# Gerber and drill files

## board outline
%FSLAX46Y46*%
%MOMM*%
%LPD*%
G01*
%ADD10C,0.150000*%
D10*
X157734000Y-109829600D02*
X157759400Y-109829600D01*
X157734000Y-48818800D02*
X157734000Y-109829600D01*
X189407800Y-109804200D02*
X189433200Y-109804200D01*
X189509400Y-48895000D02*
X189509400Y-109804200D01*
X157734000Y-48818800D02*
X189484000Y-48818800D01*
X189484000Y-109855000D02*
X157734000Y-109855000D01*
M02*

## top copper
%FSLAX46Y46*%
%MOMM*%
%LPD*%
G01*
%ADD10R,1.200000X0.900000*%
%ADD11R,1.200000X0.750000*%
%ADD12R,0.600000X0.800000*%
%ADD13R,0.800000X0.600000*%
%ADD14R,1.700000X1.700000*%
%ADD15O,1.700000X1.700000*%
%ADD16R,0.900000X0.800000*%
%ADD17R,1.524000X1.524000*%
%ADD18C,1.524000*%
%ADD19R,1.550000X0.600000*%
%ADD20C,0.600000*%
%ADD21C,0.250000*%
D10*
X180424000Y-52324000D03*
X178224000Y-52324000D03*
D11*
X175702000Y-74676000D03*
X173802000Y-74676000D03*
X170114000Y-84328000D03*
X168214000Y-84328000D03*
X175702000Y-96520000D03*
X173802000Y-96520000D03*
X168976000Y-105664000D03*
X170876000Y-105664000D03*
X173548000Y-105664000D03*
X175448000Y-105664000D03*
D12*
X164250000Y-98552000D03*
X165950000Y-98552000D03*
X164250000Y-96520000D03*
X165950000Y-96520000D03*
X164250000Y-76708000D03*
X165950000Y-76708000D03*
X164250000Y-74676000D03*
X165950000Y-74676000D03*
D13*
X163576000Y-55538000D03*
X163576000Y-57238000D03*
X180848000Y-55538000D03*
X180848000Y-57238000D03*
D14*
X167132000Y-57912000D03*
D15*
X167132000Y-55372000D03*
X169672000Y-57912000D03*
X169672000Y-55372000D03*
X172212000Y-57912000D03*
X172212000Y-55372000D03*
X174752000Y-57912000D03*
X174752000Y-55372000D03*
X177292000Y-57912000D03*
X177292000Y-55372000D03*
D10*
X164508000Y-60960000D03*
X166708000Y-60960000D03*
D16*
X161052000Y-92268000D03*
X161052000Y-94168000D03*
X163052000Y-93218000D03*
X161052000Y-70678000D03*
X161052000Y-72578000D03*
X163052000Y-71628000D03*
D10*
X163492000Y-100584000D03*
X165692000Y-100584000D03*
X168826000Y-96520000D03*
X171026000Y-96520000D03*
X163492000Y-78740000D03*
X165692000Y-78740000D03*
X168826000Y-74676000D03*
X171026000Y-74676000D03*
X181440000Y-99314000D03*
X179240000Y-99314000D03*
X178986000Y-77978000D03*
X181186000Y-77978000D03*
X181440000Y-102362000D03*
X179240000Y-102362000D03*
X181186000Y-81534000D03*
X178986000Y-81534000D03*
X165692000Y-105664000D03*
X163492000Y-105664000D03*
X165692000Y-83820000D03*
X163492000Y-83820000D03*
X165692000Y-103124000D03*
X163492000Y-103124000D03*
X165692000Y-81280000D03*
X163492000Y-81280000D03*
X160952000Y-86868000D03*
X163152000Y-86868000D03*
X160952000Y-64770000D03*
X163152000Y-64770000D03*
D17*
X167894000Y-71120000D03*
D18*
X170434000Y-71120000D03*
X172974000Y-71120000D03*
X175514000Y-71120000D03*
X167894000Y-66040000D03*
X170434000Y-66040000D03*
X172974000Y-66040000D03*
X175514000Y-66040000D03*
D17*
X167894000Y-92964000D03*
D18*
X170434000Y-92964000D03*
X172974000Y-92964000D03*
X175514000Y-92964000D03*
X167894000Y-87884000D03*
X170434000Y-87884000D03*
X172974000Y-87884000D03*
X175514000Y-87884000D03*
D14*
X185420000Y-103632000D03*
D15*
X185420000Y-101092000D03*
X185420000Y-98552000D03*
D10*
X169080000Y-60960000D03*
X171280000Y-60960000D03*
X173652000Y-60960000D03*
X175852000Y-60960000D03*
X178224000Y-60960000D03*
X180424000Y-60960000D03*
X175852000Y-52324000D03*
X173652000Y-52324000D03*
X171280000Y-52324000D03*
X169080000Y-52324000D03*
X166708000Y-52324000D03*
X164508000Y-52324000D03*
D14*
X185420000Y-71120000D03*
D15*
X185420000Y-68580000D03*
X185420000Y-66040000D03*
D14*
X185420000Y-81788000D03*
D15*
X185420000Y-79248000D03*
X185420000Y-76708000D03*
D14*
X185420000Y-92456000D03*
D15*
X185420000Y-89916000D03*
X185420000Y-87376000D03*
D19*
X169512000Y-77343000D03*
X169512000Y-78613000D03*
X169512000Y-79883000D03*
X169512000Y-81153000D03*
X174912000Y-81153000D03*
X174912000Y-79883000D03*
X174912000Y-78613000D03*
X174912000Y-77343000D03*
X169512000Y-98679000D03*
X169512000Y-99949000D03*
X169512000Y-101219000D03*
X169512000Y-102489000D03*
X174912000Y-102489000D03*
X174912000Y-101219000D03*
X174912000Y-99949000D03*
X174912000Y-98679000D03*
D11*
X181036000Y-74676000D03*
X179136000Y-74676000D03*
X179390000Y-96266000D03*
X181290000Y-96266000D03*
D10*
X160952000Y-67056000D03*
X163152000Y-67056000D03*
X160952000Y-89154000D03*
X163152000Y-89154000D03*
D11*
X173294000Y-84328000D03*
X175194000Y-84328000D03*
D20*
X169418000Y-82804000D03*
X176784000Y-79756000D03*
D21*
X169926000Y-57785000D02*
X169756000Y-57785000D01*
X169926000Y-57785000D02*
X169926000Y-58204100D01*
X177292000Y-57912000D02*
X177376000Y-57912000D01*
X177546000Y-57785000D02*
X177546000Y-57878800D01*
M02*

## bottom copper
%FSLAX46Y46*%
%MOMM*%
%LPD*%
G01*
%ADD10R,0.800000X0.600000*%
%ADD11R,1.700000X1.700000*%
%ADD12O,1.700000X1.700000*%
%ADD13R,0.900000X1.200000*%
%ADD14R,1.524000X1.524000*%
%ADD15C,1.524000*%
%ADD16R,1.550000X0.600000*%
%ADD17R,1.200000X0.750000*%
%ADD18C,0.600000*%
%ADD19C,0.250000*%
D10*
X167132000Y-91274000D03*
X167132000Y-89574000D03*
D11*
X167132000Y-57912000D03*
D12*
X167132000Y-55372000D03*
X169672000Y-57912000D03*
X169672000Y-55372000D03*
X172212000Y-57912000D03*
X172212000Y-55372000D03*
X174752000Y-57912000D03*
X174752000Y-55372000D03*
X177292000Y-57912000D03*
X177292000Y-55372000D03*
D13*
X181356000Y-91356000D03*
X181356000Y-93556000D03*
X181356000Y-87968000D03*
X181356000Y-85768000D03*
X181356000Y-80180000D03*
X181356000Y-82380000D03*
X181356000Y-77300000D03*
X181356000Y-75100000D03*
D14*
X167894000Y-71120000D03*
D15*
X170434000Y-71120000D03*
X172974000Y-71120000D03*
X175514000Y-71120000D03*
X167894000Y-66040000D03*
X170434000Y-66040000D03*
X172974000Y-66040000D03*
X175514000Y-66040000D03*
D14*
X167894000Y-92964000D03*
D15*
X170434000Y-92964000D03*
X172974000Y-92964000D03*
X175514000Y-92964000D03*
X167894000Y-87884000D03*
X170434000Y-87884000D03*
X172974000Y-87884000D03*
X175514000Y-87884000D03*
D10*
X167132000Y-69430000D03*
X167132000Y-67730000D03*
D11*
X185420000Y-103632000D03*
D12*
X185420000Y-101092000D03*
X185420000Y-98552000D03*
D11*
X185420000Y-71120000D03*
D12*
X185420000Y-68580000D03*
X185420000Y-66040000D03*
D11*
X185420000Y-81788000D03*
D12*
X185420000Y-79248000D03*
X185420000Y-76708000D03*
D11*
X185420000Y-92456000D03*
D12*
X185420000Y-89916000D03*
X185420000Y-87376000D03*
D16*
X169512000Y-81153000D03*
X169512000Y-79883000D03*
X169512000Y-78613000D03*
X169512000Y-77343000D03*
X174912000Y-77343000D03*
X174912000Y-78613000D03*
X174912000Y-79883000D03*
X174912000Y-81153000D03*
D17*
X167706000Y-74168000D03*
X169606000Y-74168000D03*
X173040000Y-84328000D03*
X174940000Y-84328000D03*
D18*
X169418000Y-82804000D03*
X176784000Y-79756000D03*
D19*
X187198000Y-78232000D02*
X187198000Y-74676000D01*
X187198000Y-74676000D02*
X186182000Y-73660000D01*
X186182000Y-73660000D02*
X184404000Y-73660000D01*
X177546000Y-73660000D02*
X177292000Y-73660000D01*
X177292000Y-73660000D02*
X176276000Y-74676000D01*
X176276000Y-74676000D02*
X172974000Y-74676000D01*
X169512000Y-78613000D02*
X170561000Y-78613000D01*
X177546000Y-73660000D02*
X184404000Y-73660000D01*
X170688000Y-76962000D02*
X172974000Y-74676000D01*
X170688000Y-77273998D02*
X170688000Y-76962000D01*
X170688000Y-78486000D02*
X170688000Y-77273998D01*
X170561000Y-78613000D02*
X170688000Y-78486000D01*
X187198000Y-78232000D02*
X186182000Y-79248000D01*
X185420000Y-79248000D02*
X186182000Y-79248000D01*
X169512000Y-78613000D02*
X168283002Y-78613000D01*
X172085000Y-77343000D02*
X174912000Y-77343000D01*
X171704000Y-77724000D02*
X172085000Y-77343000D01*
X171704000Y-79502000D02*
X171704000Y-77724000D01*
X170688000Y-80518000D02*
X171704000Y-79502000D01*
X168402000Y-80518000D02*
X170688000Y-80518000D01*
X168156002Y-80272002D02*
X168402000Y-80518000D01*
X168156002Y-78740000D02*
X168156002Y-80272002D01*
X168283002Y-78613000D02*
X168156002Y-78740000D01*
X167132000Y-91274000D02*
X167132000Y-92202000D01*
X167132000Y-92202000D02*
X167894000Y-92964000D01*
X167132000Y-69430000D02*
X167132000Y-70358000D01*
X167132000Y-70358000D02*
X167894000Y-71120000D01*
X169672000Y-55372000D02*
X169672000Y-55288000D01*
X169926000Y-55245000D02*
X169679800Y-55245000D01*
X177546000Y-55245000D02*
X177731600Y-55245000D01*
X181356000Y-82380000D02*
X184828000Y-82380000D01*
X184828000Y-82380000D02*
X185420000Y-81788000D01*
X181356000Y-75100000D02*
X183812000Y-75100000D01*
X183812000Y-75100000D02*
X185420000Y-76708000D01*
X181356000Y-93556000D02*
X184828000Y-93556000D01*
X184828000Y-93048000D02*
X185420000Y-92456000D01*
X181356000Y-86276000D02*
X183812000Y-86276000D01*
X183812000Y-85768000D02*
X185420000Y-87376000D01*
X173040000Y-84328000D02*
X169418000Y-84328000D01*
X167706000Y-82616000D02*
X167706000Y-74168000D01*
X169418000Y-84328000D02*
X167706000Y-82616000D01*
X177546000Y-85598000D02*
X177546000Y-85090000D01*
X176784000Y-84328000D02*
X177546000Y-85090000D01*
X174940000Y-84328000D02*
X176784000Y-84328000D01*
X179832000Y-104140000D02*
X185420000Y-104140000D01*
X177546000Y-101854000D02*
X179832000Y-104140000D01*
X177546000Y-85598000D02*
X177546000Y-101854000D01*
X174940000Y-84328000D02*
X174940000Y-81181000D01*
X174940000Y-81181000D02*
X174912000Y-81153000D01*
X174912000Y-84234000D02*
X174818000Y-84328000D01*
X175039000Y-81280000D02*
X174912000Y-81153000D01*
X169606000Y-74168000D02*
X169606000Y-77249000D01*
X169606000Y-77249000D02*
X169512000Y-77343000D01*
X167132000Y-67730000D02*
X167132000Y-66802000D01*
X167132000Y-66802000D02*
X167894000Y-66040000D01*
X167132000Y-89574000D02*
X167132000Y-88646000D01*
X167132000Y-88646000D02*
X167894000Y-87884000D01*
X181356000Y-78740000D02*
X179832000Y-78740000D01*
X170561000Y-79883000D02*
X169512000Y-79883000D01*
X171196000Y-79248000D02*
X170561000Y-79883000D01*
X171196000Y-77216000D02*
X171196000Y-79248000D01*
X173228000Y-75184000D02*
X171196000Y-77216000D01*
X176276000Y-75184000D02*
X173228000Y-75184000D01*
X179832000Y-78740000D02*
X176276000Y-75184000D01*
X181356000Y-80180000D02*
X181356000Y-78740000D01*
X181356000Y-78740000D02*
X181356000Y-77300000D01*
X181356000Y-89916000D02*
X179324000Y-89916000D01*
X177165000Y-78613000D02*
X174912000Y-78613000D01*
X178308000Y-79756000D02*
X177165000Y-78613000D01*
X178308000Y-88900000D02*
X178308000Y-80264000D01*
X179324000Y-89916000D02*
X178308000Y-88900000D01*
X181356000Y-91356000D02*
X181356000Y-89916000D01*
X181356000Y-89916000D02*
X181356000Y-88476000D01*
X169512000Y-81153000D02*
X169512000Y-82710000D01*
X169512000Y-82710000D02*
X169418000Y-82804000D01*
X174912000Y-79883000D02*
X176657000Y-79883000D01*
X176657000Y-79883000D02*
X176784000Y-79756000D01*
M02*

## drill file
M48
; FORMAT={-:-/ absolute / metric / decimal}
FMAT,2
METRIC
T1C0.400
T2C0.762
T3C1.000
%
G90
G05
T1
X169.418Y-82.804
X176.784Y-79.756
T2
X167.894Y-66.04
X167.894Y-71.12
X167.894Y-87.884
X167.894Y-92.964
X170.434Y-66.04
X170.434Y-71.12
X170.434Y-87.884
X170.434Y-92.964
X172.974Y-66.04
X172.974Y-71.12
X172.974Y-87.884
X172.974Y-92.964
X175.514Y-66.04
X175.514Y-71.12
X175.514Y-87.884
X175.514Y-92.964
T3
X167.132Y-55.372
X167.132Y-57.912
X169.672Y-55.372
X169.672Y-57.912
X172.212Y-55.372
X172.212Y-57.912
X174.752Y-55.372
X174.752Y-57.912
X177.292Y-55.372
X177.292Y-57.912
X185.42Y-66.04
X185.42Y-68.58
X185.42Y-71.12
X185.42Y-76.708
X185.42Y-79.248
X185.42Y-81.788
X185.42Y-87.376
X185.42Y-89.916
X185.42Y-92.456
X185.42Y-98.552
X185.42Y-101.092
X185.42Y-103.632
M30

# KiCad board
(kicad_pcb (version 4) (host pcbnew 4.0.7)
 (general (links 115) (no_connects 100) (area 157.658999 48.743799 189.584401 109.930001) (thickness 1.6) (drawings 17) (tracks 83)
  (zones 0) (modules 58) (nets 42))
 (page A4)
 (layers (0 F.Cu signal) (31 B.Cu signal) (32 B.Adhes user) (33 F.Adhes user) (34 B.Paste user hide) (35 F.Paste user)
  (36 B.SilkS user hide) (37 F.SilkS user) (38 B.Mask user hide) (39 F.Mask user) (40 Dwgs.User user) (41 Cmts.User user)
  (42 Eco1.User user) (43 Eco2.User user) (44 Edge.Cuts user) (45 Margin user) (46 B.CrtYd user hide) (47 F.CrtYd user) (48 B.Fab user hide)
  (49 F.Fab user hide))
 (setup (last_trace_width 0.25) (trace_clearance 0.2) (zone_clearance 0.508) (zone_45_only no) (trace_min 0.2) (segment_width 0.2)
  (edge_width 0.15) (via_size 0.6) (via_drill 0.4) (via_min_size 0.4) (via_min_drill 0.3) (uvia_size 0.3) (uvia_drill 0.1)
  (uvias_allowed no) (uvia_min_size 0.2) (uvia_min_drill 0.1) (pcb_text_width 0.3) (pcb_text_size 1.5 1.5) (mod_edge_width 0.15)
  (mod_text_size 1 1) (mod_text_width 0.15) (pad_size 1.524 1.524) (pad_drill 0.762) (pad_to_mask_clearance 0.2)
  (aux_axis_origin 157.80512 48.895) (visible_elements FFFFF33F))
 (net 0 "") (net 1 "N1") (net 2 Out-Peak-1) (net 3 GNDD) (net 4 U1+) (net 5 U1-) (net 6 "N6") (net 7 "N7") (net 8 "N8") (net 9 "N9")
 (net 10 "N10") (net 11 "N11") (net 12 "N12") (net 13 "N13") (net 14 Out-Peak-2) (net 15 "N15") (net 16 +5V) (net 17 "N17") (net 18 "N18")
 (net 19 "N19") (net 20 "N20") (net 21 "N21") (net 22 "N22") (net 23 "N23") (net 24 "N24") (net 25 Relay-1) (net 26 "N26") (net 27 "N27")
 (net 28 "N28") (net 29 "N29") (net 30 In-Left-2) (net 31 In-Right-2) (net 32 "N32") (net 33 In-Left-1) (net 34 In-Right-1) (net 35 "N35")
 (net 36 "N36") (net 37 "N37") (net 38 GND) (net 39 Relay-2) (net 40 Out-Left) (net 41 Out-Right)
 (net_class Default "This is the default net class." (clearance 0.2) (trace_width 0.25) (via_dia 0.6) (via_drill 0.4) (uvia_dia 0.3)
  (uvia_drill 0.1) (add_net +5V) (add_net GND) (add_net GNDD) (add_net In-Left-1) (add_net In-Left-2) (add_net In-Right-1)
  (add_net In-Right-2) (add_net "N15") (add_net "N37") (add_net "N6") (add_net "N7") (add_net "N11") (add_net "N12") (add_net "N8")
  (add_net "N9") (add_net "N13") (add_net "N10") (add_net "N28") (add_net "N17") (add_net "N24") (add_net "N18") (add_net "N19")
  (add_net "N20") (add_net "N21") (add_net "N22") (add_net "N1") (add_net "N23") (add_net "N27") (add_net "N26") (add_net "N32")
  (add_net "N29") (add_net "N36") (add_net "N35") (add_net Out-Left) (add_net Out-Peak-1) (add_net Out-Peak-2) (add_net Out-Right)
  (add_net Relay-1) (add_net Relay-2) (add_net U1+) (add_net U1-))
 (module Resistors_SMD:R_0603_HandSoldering (layer F.Cu) (at 179.324 52.324 180)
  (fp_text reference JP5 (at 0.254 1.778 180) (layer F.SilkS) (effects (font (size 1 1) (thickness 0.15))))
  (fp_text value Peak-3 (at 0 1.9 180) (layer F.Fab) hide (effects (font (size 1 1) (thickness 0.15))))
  (pad 1 smd rect (at -1.1 0 180) (size 1.2 0.9) (layers F.Cu F.Paste F.Mask) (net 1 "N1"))
  (pad 2 smd rect (at 1.1 0 180) (size 1.2 0.9) (layers F.Cu F.Paste F.Mask) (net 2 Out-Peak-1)))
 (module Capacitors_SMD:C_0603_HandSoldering (layer F.Cu) (at 174.752 74.676 180)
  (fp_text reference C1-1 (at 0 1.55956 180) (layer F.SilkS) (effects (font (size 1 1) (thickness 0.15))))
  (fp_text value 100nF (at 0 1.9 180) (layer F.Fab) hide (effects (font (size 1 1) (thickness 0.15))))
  (pad 1 smd rect (at -0.95 0 180) (size 1.2 0.75) (layers F.Cu F.Paste F.Mask) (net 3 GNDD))
  (pad 2 smd rect (at 0.95 0 180) (size 1.2 0.75) (layers F.Cu F.Paste F.Mask) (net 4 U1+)))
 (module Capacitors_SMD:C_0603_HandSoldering (layer F.Cu) (at 169.164 84.328 180)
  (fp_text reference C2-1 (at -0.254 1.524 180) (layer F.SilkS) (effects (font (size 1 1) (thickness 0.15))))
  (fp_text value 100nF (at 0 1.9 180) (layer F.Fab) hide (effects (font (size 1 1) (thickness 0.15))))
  (pad 1 smd rect (at -0.95 0 180) (size 1.2 0.75) (layers F.Cu F.Paste F.Mask) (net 3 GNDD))
  (pad 2 smd rect (at 0.95 0 180) (size 1.2 0.75) (layers F.Cu F.Paste F.Mask) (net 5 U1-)))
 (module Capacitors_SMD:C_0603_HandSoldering (layer F.Cu) (at 174.752 96.52 180)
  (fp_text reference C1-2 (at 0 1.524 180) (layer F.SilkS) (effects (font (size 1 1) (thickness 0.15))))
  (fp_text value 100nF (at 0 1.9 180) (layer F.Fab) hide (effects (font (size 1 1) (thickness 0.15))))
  (pad 1 smd rect (at -0.95 0 180) (size 1.2 0.75) (layers F.Cu F.Paste F.Mask) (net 3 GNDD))
  (pad 2 smd rect (at 0.95 0 180) (size 1.2 0.75) (layers F.Cu F.Paste F.Mask) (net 4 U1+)))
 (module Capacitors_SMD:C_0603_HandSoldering (layer F.Cu) (at 169.926 105.664)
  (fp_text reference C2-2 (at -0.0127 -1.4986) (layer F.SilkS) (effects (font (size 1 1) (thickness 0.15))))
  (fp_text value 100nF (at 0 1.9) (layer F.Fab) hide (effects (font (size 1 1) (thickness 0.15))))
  (pad 1 smd rect (at -0.95 0) (size 1.2 0.75) (layers F.Cu F.Paste F.Mask) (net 3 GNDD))
  (pad 2 smd rect (at 0.95 0) (size 1.2 0.75) (layers F.Cu F.Paste F.Mask) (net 5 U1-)))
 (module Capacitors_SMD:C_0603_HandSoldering (layer F.Cu) (at 174.498 105.664)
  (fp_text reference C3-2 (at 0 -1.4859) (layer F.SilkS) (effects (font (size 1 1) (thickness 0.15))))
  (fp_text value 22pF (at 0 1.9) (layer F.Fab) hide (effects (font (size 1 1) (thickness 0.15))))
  (pad 1 smd rect (at -0.95 0) (size 1.2 0.75) (layers F.Cu F.Paste F.Mask) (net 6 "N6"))
  (pad 2 smd rect (at 0.95 0) (size 1.2 0.75) (layers F.Cu F.Paste F.Mask) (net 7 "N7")))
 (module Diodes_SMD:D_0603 (layer F.Cu) (at 165.1 98.552)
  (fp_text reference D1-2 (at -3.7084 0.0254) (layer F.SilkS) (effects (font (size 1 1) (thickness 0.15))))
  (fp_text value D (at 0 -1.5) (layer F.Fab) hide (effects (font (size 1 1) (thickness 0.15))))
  (pad 1 smd rect (at -0.85 0) (size 0.6 0.8) (layers F.Cu F.Paste F.Mask) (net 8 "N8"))
  (pad 2 smd rect (at 0.85 0) (size 0.6 0.8) (layers F.Cu F.Paste F.Mask) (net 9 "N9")))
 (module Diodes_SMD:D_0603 (layer F.Cu) (at 165.1 96.52)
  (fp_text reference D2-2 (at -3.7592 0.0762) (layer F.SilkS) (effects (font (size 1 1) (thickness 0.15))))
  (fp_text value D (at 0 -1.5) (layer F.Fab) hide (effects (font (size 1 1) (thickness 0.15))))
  (pad 1 smd rect (at -0.85 0) (size 0.6 0.8) (layers F.Cu F.Paste F.Mask) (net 9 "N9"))
  (pad 2 smd rect (at 0.85 0) (size 0.6 0.8) (layers F.Cu F.Paste F.Mask) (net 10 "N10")))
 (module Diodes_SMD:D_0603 (layer F.Cu) (at 165.1 76.708)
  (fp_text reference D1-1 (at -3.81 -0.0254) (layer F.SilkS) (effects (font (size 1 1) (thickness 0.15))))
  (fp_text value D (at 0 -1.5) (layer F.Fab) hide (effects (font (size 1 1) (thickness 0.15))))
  (pad 1 smd rect (at -0.85 0) (size 0.6 0.8) (layers F.Cu F.Paste F.Mask) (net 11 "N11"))
  (pad 2 smd rect (at 0.85 0) (size 0.6 0.8) (layers F.Cu F.Paste F.Mask) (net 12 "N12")))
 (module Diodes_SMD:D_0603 (layer F.Cu) (at 165.1 74.676)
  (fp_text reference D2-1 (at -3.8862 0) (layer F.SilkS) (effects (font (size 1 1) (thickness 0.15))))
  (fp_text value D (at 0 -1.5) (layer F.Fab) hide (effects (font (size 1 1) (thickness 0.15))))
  (pad 1 smd rect (at -0.85 0) (size 0.6 0.8) (layers F.Cu F.Paste F.Mask) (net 12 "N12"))
  (pad 2 smd rect (at 0.85 0) (size 0.6 0.8) (layers F.Cu F.Paste F.Mask) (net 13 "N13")))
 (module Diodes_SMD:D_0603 (layer F.Cu) (at 163.576 56.388 270)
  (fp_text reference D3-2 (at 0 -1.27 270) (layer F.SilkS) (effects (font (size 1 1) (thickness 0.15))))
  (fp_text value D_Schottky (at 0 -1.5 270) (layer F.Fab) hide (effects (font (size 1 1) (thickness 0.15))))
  (pad 1 smd rect (at -0.85 0 270) (size 0.6 0.8) (layers F.Cu F.Paste F.Mask) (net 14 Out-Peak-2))
  (pad 2 smd rect (at 0.85 0 270) (size 0.6 0.8) (layers F.Cu F.Paste F.Mask) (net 6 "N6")))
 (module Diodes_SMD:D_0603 (layer F.Cu) (at 180.848 56.388 270)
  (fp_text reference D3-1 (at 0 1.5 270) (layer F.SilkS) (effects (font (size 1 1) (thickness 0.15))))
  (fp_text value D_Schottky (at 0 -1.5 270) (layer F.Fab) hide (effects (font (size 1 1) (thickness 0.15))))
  (pad 1 smd rect (at -0.85 0 270) (size 0.6 0.8) (layers F.Cu F.Paste F.Mask) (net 2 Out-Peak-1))
  (pad 2 smd rect (at 0.85 0 270) (size 0.6 0.8) (layers F.Cu F.Paste F.Mask) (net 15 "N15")))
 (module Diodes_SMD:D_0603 (layer B.Cu) (at 167.132 90.424 90)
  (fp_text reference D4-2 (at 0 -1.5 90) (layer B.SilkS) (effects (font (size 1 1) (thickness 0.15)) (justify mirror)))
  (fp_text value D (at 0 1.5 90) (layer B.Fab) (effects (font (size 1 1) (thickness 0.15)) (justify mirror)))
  (pad 1 smd rect (at -0.85 0 90) (size 0.6 0.8) (layers B.Cu B.Paste B.Mask) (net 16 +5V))
  (pad 2 smd rect (at 0.85 0 90) (size 0.6 0.8) (layers B.Cu B.Paste B.Mask) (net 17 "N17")))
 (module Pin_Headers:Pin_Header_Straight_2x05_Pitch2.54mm (layer F.Cu) (at 167.132 57.912 90)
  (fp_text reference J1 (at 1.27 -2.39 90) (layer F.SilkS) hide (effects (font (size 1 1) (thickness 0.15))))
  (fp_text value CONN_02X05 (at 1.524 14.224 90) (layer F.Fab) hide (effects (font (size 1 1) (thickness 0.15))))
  (pad 1 thru_hole rect (at 0 0 90) (size 1.7 1.7) (drill 1) (layers *.Cu *.Mask) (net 16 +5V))
  (pad 2 thru_hole oval (at 2.54 0 90) (size 1.7 1.7) (drill 1) (layers *.Cu *.Mask) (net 3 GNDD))
  (pad 3 thru_hole oval (at 0 2.54 90) (size 1.7 1.7) (drill 1) (layers *.Cu *.Mask) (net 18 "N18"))
  (pad 4 thru_hole oval (at 2.54 2.54 90) (size 1.7 1.7) (drill 1) (layers *.Cu *.Mask) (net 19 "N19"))
  (pad 5 thru_hole oval (at 0 5.08 90) (size 1.7 1.7) (drill 1) (layers *.Cu *.Mask) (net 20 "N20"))
  (pad 6 thru_hole oval (at 2.54 5.08 90) (size 1.7 1.7) (drill 1) (layers *.Cu *.Mask) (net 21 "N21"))
  (pad 7 thru_hole oval (at 0 7.62 90) (size 1.7 1.7) (drill 1) (layers *.Cu *.Mask) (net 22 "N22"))
  (pad 8 thru_hole oval (at 2.54 7.62 90) (size 1.7 1.7) (drill 1) (layers *.Cu *.Mask) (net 1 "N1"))
  (pad 9 thru_hole oval (at 0 10.16 90) (size 1.7 1.7) (drill 1) (layers *.Cu *.Mask) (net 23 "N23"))
  (pad 10 thru_hole oval (at 2.54 10.16 90) (size 1.7 1.7) (drill 1) (layers *.Cu *.Mask) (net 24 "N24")))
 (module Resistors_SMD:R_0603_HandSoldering (layer F.Cu) (at 165.608 60.96)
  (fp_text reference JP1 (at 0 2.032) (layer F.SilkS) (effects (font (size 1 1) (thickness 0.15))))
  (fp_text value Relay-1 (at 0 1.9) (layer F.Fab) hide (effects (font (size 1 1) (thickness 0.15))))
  (pad 1 smd rect (at -1.1 0) (size 1.2 0.9) (layers F.Cu F.Paste F.Mask) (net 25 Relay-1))
  (pad 2 smd rect (at 1.1 0) (size 1.2 0.9) (layers F.Cu F.Paste F.Mask) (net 18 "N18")))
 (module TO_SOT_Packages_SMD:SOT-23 (layer F.Cu) (at 162.052 93.218)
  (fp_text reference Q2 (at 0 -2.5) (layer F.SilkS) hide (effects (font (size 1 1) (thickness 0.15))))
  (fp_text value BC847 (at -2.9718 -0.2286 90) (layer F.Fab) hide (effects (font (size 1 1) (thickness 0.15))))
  (pad 1 smd rect (at -1 -0.95) (size 0.9 0.8) (layers F.Cu F.Paste F.Mask) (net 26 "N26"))
  (pad 2 smd rect (at -1 0.95) (size 0.9 0.8) (layers F.Cu F.Paste F.Mask) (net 3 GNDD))
  (pad 3 smd rect (at 1 0) (size 0.9 0.8) (layers F.Cu F.Paste F.Mask) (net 17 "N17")))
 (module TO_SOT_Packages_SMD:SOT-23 (layer F.Cu) (at 162.052 71.628)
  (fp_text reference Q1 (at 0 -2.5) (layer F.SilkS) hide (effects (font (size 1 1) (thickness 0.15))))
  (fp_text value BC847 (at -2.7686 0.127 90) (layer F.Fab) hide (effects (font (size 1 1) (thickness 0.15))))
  (pad 1 smd rect (at -1 -0.95) (size 0.9 0.8) (layers F.Cu F.Paste F.Mask) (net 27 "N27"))
  (pad 2 smd rect (at -1 0.95) (size 0.9 0.8) (layers F.Cu F.Paste F.Mask) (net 3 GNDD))
  (pad 3 smd rect (at 1 0) (size 0.9 0.8) (layers F.Cu F.Paste F.Mask) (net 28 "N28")))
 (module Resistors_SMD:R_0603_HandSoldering (layer B.Cu) (at 181.356 92.456 270)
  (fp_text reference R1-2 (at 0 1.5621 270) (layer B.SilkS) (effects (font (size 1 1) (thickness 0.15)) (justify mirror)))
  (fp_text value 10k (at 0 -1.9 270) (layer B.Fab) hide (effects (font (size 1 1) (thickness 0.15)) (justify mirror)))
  (pad 1 smd rect (at -1.1 0 270) (size 1.2 0.9) (layers B.Cu B.Paste B.Mask) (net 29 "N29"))
  (pad 2 smd rect (at 1.1 0 270) (size 1.2 0.9) (layers B.Cu B.Paste B.Mask) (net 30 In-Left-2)))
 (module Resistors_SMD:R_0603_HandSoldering (layer B.Cu) (at 181.356 86.868 90)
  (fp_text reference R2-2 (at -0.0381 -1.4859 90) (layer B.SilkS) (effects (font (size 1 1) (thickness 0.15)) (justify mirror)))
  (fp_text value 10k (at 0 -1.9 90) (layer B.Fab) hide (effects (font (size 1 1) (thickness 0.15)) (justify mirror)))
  (pad 1 smd rect (at -1.1 0 90) (size 1.2 0.9) (layers B.Cu B.Paste B.Mask) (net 29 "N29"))
  (pad 2 smd rect (at 1.1 0 90) (size 1.2 0.9) (layers B.Cu B.Paste B.Mask) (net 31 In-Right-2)))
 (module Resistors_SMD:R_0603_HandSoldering (layer B.Cu) (at 181.356 81.28 270)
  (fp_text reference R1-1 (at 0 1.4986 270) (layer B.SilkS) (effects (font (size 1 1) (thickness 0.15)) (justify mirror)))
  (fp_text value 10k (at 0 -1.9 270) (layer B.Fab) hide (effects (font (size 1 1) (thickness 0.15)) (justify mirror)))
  (pad 1 smd rect (at -1.1 0 270) (size 1.2 0.9) (layers B.Cu B.Paste B.Mask) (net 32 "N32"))
  (pad 2 smd rect (at 1.1 0 270) (size 1.2 0.9) (layers B.Cu B.Paste B.Mask) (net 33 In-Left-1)))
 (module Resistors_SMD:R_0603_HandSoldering (layer B.Cu) (at 181.356 76.2 90)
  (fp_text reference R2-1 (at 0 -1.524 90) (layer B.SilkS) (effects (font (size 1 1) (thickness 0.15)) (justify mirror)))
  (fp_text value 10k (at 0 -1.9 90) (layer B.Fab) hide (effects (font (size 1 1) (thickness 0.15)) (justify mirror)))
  (pad 1 smd rect (at -1.1 0 90) (size 1.2 0.9) (layers B.Cu B.Paste B.Mask) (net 32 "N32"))
  (pad 2 smd rect (at 1.1 0 90) (size 1.2 0.9) (layers B.Cu B.Paste B.Mask) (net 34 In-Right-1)))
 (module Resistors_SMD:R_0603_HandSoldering (layer F.Cu) (at 164.592 100.584)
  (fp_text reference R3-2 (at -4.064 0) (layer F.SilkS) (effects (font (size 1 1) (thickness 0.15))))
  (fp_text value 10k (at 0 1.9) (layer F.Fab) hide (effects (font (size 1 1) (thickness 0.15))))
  (pad 1 smd rect (at -1.1 0) (size 1.2 0.9) (layers F.Cu F.Paste F.Mask) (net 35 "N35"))
  (pad 2 smd rect (at 1.1 0) (size 1.2 0.9) (layers F.Cu F.Paste F.Mask) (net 29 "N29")))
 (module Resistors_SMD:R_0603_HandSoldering (layer F.Cu) (at 169.926 96.52)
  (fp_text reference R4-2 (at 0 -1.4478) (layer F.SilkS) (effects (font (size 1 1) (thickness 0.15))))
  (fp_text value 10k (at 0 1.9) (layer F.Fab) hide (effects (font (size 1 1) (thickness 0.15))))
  (pad 1 smd rect (at -1.1 0) (size 1.2 0.9) (layers F.Cu F.Paste F.Mask) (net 8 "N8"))
  (pad 2 smd rect (at 1.1 0) (size 1.2 0.9) (layers F.Cu F.Paste F.Mask) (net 35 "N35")))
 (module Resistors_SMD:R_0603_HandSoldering (layer F.Cu) (at 164.592 78.74)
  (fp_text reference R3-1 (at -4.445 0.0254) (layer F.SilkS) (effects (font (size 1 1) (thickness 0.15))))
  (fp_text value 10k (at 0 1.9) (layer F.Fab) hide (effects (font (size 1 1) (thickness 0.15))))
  (pad 1 smd rect (at -1.1 0) (size 1.2 0.9) (layers F.Cu F.Paste F.Mask) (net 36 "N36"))
  (pad 2 smd rect (at 1.1 0) (size 1.2 0.9) (layers F.Cu F.Paste F.Mask) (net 32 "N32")))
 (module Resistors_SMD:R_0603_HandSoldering (layer F.Cu) (at 169.926 74.676)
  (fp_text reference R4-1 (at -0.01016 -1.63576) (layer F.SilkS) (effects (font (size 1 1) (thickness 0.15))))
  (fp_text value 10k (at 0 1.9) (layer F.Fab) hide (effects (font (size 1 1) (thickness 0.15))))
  (pad 1 smd rect (at -1.1 0) (size 1.2 0.9) (layers F.Cu F.Paste F.Mask) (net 11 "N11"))
  (pad 2 smd rect (at 1.1 0) (size 1.2 0.9) (layers F.Cu F.Paste F.Mask) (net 36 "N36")))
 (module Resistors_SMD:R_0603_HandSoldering (layer F.Cu) (at 180.34 99.314 180)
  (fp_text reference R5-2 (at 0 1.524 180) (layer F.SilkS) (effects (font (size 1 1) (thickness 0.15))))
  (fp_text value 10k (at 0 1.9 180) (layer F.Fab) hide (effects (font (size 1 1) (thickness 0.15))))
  (pad 1 smd rect (at -1.1 0 180) (size 1.2 0.9) (layers F.Cu F.Paste F.Mask) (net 10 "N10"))
  (pad 2 smd rect (at 1.1 0 180) (size 1.2 0.9) (layers F.Cu F.Paste F.Mask) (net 35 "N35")))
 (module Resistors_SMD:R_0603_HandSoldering (layer F.Cu) (at 180.086 77.978)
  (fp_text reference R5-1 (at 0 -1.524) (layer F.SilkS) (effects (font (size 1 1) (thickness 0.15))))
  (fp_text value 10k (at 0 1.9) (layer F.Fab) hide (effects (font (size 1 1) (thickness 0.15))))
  (pad 1 smd rect (at -1.1 0) (size 1.2 0.9) (layers F.Cu F.Paste F.Mask) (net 13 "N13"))
  (pad 2 smd rect (at 1.1 0) (size 1.2 0.9) (layers F.Cu F.Paste F.Mask) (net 36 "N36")))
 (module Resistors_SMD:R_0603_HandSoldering (layer F.Cu) (at 180.34 102.362 180)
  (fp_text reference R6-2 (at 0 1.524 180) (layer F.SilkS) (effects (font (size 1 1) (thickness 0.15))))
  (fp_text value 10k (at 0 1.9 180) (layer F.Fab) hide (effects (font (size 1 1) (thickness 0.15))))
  (pad 1 smd rect (at -1.1 0 180) (size 1.2 0.9) (layers F.Cu F.Paste F.Mask) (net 7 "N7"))
  (pad 2 smd rect (at 1.1 0 180) (size 1.2 0.9) (layers F.Cu F.Paste F.Mask) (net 10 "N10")))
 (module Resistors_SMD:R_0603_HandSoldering (layer F.Cu) (at 180.086 81.534 180)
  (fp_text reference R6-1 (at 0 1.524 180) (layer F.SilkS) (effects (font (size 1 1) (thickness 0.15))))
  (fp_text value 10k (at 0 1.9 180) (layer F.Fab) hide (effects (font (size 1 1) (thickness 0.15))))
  (pad 1 smd rect (at -1.1 0 180) (size 1.2 0.9) (layers F.Cu F.Paste F.Mask) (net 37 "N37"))
  (pad 2 smd rect (at 1.1 0 180) (size 1.2 0.9) (layers F.Cu F.Paste F.Mask) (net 13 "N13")))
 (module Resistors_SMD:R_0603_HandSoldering (layer F.Cu) (at 164.592 105.664 180)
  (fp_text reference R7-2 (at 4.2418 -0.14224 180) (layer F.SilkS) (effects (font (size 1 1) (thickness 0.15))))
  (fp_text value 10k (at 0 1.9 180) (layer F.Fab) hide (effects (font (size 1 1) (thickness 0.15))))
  (pad 1 smd rect (at -1.1 0 180) (size 1.2 0.9) (layers F.Cu F.Paste F.Mask) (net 6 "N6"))
  (pad 2 smd rect (at 1.1 0 180) (size 1.2 0.9) (layers F.Cu F.Paste F.Mask) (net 7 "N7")))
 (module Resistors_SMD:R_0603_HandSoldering (layer F.Cu) (at 164.592 83.82 180)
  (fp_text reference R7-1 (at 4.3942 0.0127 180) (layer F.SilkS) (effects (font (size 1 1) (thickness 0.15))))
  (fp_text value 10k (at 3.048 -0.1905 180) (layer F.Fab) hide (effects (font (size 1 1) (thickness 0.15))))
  (pad 1 smd rect (at -1.1 0 180) (size 1.2 0.9) (layers F.Cu F.Paste F.Mask) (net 15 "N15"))
  (pad 2 smd rect (at 1.1 0 180) (size 1.2 0.9) (layers F.Cu F.Paste F.Mask) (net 37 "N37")))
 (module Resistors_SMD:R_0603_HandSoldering (layer F.Cu) (at 164.592 103.124 180)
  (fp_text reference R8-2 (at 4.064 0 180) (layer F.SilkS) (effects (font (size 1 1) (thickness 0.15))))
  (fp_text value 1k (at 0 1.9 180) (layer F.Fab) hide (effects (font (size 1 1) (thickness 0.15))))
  (pad 1 smd rect (at -1.1 0 180) (size 1.2 0.9) (layers F.Cu F.Paste F.Mask) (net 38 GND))
  (pad 2 smd rect (at 1.1 0 180) (size 1.2 0.9) (layers F.Cu F.Paste F.Mask) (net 14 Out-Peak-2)))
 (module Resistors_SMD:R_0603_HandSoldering (layer F.Cu) (at 164.592 81.28 180)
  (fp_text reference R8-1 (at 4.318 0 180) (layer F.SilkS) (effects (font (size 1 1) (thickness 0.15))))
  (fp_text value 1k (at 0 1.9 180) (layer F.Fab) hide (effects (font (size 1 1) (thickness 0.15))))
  (pad 1 smd rect (at -1.1 0 180) (size 1.2 0.9) (layers F.Cu F.Paste F.Mask) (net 38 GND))
  (pad 2 smd rect (at 1.1 0 180) (size 1.2 0.9) (layers F.Cu F.Paste F.Mask) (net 2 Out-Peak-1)))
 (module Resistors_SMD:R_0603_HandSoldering (layer F.Cu) (at 162.052 86.868)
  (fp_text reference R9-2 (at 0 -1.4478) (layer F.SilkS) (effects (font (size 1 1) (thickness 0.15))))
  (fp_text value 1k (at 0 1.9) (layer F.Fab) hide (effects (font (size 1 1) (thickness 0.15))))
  (pad 1 smd rect (at -1.1 0) (size 1.2 0.9) (layers F.Cu F.Paste F.Mask) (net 26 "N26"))
  (pad 2 smd rect (at 1.1 0) (size 1.2 0.9) (layers F.Cu F.Paste F.Mask) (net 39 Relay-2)))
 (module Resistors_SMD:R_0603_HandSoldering (layer F.Cu) (at 162.052 64.77)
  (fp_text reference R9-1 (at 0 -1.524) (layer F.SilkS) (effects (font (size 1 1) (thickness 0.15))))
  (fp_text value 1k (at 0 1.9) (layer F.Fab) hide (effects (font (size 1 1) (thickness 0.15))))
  (pad 1 smd rect (at -1.1 0) (size 1.2 0.9) (layers F.Cu F.Paste F.Mask) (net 27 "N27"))
  (pad 2 smd rect (at 1.1 0) (size 1.2 0.9) (layers F.Cu F.Paste F.Mask) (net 25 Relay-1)))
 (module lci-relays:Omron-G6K (layer F.Cu) (at 171.704 68.58)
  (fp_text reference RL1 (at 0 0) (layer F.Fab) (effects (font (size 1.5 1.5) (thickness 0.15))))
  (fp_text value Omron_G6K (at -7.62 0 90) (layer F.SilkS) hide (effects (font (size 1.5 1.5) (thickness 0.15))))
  (pad 1 thru_hole rect (at -3.81 2.54) (size 1.524 1.524) (drill 0.762) (layers *.Cu *.Mask F.SilkS) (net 16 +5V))
  (pad 2 thru_hole circle (at -1.27 2.54) (size 1.524 1.524) (drill 0.762) (layers *.Cu *.Mask F.SilkS))
  (pad 3 thru_hole circle (at 1.27 2.54) (size 1.524 1.524) (drill 0.762) (layers *.Cu *.Mask F.SilkS) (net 33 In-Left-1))
  (pad 4 thru_hole circle (at 3.81 2.54) (size 1.524 1.524) (drill 0.762) (layers *.Cu *.Mask F.SilkS) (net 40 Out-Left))
  (pad 8 thru_hole circle (at -3.81 -2.54) (size 1.524 1.524) (drill 0.762) (layers *.Cu *.Mask F.SilkS) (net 28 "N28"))
  (pad 7 thru_hole circle (at -1.27 -2.54) (size 1.524 1.524) (drill 0.762) (layers *.Cu *.Mask F.SilkS))
  (pad 6 thru_hole circle (at 1.27 -2.54) (size 1.524 1.524) (drill 0.762) (layers *.Cu *.Mask F.SilkS) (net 34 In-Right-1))
  (pad 5 thru_hole circle (at 3.81 -2.54) (size 1.524 1.524) (drill 0.762) (layers *.Cu *.Mask F.SilkS) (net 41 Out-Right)))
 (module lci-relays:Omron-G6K (layer F.Cu) (at 171.704 90.424)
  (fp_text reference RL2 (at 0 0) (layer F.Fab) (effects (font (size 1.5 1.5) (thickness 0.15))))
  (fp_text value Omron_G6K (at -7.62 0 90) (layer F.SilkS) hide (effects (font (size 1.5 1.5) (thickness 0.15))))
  (pad 1 thru_hole rect (at -3.81 2.54) (size 1.524 1.524) (drill 0.762) (layers *.Cu *.Mask F.SilkS) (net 16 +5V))
  (pad 2 thru_hole circle (at -1.27 2.54) (size 1.524 1.524) (drill 0.762) (layers *.Cu *.Mask F.SilkS))
  (pad 3 thru_hole circle (at 1.27 2.54) (size 1.524 1.524) (drill 0.762) (layers *.Cu *.Mask F.SilkS) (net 30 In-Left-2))
  (pad 4 thru_hole circle (at 3.81 2.54) (size 1.524 1.524) (drill 0.762) (layers *.Cu *.Mask F.SilkS) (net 40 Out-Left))
  (pad 8 thru_hole circle (at -3.81 -2.54) (size 1.524 1.524) (drill 0.762) (layers *.Cu *.Mask F.SilkS) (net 17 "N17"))
  (pad 7 thru_hole circle (at -1.27 -2.54) (size 1.524 1.524) (drill 0.762) (layers *.Cu *.Mask F.SilkS))
  (pad 6 thru_hole circle (at 1.27 -2.54) (size 1.524 1.524) (drill 0.762) (layers *.Cu *.Mask F.SilkS) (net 31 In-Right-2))
  (pad 5 thru_hole circle (at 3.81 -2.54) (size 1.524 1.524) (drill 0.762) (layers *.Cu *.Mask F.SilkS) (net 41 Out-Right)))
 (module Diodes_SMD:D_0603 (layer B.Cu) (at 167.132 68.58 90)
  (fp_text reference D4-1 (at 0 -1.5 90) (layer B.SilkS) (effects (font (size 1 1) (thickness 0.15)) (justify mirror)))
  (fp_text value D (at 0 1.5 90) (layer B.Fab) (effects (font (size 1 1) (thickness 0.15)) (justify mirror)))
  (pad 1 smd rect (at -0.85 0 90) (size 0.6 0.8) (layers B.Cu B.Paste B.Mask) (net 16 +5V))
  (pad 2 smd rect (at 0.85 0 90) (size 0.6 0.8) (layers B.Cu B.Paste B.Mask) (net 28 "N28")))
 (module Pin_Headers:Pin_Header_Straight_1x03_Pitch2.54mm (layer F.Cu) (at 185.42 103.632 180)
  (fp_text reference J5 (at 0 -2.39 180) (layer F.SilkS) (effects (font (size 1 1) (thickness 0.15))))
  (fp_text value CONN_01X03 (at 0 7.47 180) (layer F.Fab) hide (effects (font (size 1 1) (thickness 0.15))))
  (pad 1 thru_hole rect (at 0 0 180) (size 1.7 1.7) (drill 1) (layers *.Cu *.Mask) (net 4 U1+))
  (pad 2 thru_hole oval (at 0 2.54 180) (size 1.7 1.7) (drill 1) (layers *.Cu *.Mask) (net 3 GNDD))
  (pad 3 thru_hole oval (at 0 5.08 180) (size 1.7 1.7) (drill 1) (layers *.Cu *.Mask) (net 5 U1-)))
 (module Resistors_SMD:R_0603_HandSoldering (layer F.Cu) (at 170.18 60.96)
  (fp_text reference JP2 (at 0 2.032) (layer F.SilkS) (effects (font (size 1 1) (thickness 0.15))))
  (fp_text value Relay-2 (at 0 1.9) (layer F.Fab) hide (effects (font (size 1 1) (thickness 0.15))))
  (pad 1 smd rect (at -1.1 0) (size 1.2 0.9) (layers F.Cu F.Paste F.Mask) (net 39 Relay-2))
  (pad 2 smd rect (at 1.1 0) (size 1.2 0.9) (layers F.Cu F.Paste F.Mask) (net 20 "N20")))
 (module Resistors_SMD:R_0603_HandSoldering (layer F.Cu) (at 174.752 60.96)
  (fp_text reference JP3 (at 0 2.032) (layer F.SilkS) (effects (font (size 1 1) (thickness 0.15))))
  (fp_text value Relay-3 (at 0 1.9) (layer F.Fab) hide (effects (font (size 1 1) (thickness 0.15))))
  (pad 1 smd rect (at -1.1 0) (size 1.2 0.9) (layers F.Cu F.Paste F.Mask) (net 25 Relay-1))
  (pad 2 smd rect (at 1.1 0) (size 1.2 0.9) (layers F.Cu F.Paste F.Mask) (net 22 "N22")))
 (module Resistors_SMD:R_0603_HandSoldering (layer F.Cu) (at 179.324 60.96)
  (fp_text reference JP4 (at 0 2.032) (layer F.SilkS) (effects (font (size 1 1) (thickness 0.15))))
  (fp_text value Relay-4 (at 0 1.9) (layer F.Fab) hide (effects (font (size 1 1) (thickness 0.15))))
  (pad 1 smd rect (at -1.1 0) (size 1.2 0.9) (layers F.Cu F.Paste F.Mask) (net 39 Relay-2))
  (pad 2 smd rect (at 1.1 0) (size 1.2 0.9) (layers F.Cu F.Paste F.Mask) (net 23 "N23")))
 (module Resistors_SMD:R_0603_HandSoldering (layer F.Cu) (at 174.752 52.324 180)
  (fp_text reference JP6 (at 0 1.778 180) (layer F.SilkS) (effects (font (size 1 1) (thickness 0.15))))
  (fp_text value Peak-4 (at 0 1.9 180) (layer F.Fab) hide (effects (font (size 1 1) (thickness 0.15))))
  (pad 1 smd rect (at -1.1 0 180) (size 1.2 0.9) (layers F.Cu F.Paste F.Mask) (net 24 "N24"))
  (pad 2 smd rect (at 1.1 0 180) (size 1.2 0.9) (layers F.Cu F.Paste F.Mask) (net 14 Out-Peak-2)))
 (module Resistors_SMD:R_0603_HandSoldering (layer F.Cu) (at 170.18 52.324 180)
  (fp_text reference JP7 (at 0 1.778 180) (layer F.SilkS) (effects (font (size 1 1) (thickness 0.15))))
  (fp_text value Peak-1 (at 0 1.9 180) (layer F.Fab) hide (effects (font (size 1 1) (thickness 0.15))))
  (pad 1 smd rect (at -1.1 0 180) (size 1.2 0.9) (layers F.Cu F.Paste F.Mask) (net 19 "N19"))
  (pad 2 smd rect (at 1.1 0 180) (size 1.2 0.9) (layers F.Cu F.Paste F.Mask) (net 2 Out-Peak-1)))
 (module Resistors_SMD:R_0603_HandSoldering (layer F.Cu) (at 165.608 52.324 180)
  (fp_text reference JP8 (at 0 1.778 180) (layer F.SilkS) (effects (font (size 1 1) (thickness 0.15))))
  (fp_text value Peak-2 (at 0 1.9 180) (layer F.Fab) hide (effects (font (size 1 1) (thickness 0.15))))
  (pad 1 smd rect (at -1.1 0 180) (size 1.2 0.9) (layers F.Cu F.Paste F.Mask) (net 21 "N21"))
  (pad 2 smd rect (at 1.1 0 180) (size 1.2 0.9) (layers F.Cu F.Paste F.Mask) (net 14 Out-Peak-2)))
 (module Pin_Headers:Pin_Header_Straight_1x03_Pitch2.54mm (layer F.Cu) (at 185.42 71.12 180)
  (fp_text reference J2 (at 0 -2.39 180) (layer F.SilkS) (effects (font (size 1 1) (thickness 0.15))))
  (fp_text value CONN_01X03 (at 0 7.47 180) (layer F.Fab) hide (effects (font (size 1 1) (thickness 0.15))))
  (pad 1 thru_hole rect (at 0 0 180) (size 1.7 1.7) (drill 1) (layers *.Cu *.Mask) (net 41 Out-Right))
  (pad 2 thru_hole oval (at 0 2.54 180) (size 1.7 1.7) (drill 1) (layers *.Cu *.Mask) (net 38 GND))
  (pad 3 thru_hole oval (at 0 5.08 180) (size 1.7 1.7) (drill 1) (layers *.Cu *.Mask) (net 40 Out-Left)))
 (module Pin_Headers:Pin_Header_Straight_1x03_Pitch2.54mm (layer F.Cu) (at 185.42 81.788 180)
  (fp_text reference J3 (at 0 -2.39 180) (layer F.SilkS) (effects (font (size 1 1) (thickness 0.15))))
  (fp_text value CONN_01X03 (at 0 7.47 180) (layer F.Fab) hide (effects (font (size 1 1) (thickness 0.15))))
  (pad 1 thru_hole rect (at 0 0 180) (size 1.7 1.7) (drill 1) (layers *.Cu *.Mask) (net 33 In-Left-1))
  (pad 2 thru_hole oval (at 0 2.54 180) (size 1.7 1.7) (drill 1) (layers *.Cu *.Mask) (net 38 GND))
  (pad 3 thru_hole oval (at 0 5.08 180) (size 1.7 1.7) (drill 1) (layers *.Cu *.Mask) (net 34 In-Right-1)))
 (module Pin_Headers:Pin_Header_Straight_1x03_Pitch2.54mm (layer F.Cu) (at 185.42 92.456 180)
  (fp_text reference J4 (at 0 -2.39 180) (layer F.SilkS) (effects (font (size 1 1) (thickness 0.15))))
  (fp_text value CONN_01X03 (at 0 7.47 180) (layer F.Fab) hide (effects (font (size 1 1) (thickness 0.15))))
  (pad 1 thru_hole rect (at 0 0 180) (size 1.7 1.7) (drill 1) (layers *.Cu *.Mask) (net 30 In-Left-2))
  (pad 2 thru_hole oval (at 0 2.54 180) (size 1.7 1.7) (drill 1) (layers *.Cu *.Mask) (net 38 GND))
  (pad 3 thru_hole oval (at 0 5.08 180) (size 1.7 1.7) (drill 1) (layers *.Cu *.Mask) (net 31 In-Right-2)))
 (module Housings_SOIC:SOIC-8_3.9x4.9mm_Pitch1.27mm (layer B.Cu) (at 172.212 79.248)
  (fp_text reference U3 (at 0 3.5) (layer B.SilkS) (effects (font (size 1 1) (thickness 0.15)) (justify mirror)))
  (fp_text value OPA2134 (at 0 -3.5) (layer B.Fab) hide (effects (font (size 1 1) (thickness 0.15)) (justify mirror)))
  (pad 1 smd rect (at -2.7 1.905) (size 1.55 0.6) (layers B.Cu B.Paste B.Mask) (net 36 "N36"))
  (pad 2 smd rect (at -2.7 0.635) (size 1.55 0.6) (layers B.Cu B.Paste B.Mask) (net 32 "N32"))
  (pad 3 smd rect (at -2.7 -0.635) (size 1.55 0.6) (layers B.Cu B.Paste B.Mask) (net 38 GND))
  (pad 4 smd rect (at -2.7 -1.905) (size 1.55 0.6) (layers B.Cu B.Paste B.Mask) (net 5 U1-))
  (pad 5 smd rect (at 2.7 -1.905) (size 1.55 0.6) (layers B.Cu B.Paste B.Mask) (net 38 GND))
  (pad 6 smd rect (at 2.7 -0.635) (size 1.55 0.6) (layers B.Cu B.Paste B.Mask) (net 29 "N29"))
  (pad 7 smd rect (at 2.7 0.635) (size 1.55 0.6) (layers B.Cu B.Paste B.Mask) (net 35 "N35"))
  (pad 8 smd rect (at 2.7 1.905) (size 1.55 0.6) (layers B.Cu B.Paste B.Mask) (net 4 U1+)))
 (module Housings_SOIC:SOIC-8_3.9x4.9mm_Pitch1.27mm (layer F.Cu) (at 172.212 79.248)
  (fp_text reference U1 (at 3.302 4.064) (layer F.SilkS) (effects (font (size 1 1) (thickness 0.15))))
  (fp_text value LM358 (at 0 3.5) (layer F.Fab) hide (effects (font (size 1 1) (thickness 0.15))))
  (pad 1 smd rect (at -2.7 -1.905) (size 1.55 0.6) (layers F.Cu F.Paste F.Mask) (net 12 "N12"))
  (pad 2 smd rect (at -2.7 -0.635) (size 1.55 0.6) (layers F.Cu F.Paste F.Mask) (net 36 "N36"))
  (pad 3 smd rect (at -2.7 0.635) (size 1.55 0.6) (layers F.Cu F.Paste F.Mask) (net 38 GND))
  (pad 4 smd rect (at -2.7 1.905) (size 1.55 0.6) (layers F.Cu F.Paste F.Mask) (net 5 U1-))
  (pad 5 smd rect (at 2.7 1.905) (size 1.55 0.6) (layers F.Cu F.Paste F.Mask) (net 11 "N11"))
  (pad 6 smd rect (at 2.7 0.635) (size 1.55 0.6) (layers F.Cu F.Paste F.Mask) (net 37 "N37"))
  (pad 7 smd rect (at 2.7 -0.635) (size 1.55 0.6) (layers F.Cu F.Paste F.Mask) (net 15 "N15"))
  (pad 8 smd rect (at 2.7 -1.905) (size 1.55 0.6) (layers F.Cu F.Paste F.Mask) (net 4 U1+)))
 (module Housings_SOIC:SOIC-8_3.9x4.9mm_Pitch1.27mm (layer F.Cu) (at 172.212 100.584)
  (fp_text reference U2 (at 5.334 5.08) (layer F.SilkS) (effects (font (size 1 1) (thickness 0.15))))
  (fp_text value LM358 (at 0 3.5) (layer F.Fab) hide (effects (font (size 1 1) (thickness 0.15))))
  (pad 1 smd rect (at -2.7 -1.905) (size 1.55 0.6) (layers F.Cu F.Paste F.Mask) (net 9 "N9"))
  (pad 2 smd rect (at -2.7 -0.635) (size 1.55 0.6) (layers F.Cu F.Paste F.Mask) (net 35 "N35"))
  (pad 3 smd rect (at -2.7 0.635) (size 1.55 0.6) (layers F.Cu F.Paste F.Mask) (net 38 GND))
  (pad 4 smd rect (at -2.7 1.905) (size 1.55 0.6) (layers F.Cu F.Paste F.Mask) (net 5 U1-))
  (pad 5 smd rect (at 2.7 1.905) (size 1.55 0.6) (layers F.Cu F.Paste F.Mask) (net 8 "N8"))
  (pad 6 smd rect (at 2.7 0.635) (size 1.55 0.6) (layers F.Cu F.Paste F.Mask) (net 7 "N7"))
  (pad 7 smd rect (at 2.7 -0.635) (size 1.55 0.6) (layers F.Cu F.Paste F.Mask) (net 6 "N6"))
  (pad 8 smd rect (at 2.7 -1.905) (size 1.55 0.6) (layers F.Cu F.Paste F.Mask) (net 4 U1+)))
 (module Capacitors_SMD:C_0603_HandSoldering (layer B.Cu) (at 168.656 74.168)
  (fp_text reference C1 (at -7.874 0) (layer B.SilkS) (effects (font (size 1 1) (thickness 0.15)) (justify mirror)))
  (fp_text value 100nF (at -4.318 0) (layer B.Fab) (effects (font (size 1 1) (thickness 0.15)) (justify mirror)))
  (pad 1 smd rect (at -0.95 0) (size 1.2 0.75) (layers B.Cu B.Paste B.Mask) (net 3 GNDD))
  (pad 2 smd rect (at 0.95 0) (size 1.2 0.75) (layers B.Cu B.Paste B.Mask) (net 5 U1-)))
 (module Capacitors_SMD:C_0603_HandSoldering (layer B.Cu) (at 173.99 84.328)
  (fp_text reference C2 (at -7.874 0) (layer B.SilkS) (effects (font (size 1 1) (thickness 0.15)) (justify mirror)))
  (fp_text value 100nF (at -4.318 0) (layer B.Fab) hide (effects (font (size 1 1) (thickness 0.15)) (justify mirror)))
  (pad 1 smd rect (at -0.95 0) (size 1.2 0.75) (layers B.Cu B.Paste B.Mask) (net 3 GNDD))
  (pad 2 smd rect (at 0.95 0) (size 1.2 0.75) (layers B.Cu B.Paste B.Mask) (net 4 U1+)))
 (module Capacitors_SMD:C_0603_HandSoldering (layer F.Cu) (at 180.086 74.676 180)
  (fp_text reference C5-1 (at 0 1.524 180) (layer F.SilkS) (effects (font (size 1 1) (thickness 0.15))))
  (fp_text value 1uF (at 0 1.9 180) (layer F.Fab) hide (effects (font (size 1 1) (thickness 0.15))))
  (pad 1 smd rect (at -0.95 0 180) (size 1.2 0.75) (layers F.Cu F.Paste F.Mask) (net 38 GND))
  (pad 2 smd rect (at 0.95 0 180) (size 1.2 0.75) (layers F.Cu F.Paste F.Mask) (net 2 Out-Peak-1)))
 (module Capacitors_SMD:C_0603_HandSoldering (layer F.Cu) (at 180.34 96.266)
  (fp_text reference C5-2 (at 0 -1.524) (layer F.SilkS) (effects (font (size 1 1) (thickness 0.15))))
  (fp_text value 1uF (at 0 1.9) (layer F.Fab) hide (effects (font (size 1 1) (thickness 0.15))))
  (pad 1 smd rect (at -0.95 0) (size 1.2 0.75) (layers F.Cu F.Paste F.Mask) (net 38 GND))
  (pad 2 smd rect (at 0.95 0) (size 1.2 0.75) (layers F.Cu F.Paste F.Mask) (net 14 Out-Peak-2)))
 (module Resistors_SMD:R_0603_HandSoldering (layer F.Cu) (at 162.052 67.056)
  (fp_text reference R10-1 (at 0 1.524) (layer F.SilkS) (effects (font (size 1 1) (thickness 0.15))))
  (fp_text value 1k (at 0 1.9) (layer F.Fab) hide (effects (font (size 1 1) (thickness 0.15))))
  (pad 1 smd rect (at -1.1 0) (size 1.2 0.9) (layers F.Cu F.Paste F.Mask) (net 3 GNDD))
  (pad 2 smd rect (at 1.1 0) (size 1.2 0.9) (layers F.Cu F.Paste F.Mask) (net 27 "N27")))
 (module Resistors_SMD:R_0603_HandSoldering (layer F.Cu) (at 162.052 89.154)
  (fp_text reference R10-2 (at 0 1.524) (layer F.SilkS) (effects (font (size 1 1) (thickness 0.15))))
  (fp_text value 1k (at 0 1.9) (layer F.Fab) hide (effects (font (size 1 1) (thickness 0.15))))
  (pad 1 smd rect (at -1.1 0) (size 1.2 0.9) (layers F.Cu F.Paste F.Mask) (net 3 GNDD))
  (pad 2 smd rect (at 1.1 0) (size 1.2 0.9) (layers F.Cu F.Paste F.Mask) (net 26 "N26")))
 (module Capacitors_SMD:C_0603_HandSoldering (layer F.Cu) (at 174.244 84.328)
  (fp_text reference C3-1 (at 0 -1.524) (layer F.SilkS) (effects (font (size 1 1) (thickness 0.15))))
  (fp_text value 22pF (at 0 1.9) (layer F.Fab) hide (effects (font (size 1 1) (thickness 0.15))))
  (pad 1 smd rect (at -0.95 0) (size 1.2 0.75) (layers F.Cu F.Paste F.Mask) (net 15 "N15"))
  (pad 2 smd rect (at 0.95 0) (size 1.2 0.75) (layers F.Cu F.Paste F.Mask) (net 37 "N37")))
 (gr_line (start 157.734 109.8296) (end 157.7594 109.8296) (angle 90) (layer Edge.Cuts) (width 0.15))
 (gr_line (start 157.734 48.8188) (end 157.734 109.8296) (angle 90) (layer Edge.Cuts) (width 0.15))
 (gr_line (start 189.4078 109.8042) (end 189.4332 109.8042) (angle 90) (layer Edge.Cuts) (width 0.15))
 (gr_line (start 189.5094 48.895) (end 189.5094 109.8042) (angle 90) (layer Edge.Cuts) (width 0.15))
 (gr_line (start 157.734 48.8188) (end 189.484 48.8188) (angle 90) (layer Edge.Cuts) (width 0.15))
 (gr_line (start 189.484 109.855) (end 157.734 109.855) (angle 90) (layer Edge.Cuts) (width 0.15))
 (segment (start 187.198 78.232) (end 187.198 74.676) (width 0.25) (layer B.Cu) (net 38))
 (segment (start 187.198 74.676) (end 186.182 73.66) (width 0.25) (layer B.Cu) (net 38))
 (segment (start 186.182 73.66) (end 184.404 73.66) (width 0.25) (layer B.Cu) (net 38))
 (segment (start 177.546 73.66) (end 177.292 73.66) (width 0.25) (layer B.Cu) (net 38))
 (segment (start 177.292 73.66) (end 176.276 74.676) (width 0.25) (layer B.Cu) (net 38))
 (segment (start 176.276 74.676) (end 172.974 74.676) (width 0.25) (layer B.Cu) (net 38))
 (segment (start 169.512 78.613) (end 170.561 78.613) (width 0.25) (layer B.Cu) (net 38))
 (segment (start 177.546 73.66) (end 184.404 73.66) (width 0.25) (layer B.Cu) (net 38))
 (segment (start 170.688 76.962) (end 172.974 74.676) (width 0.25) (layer B.Cu) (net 38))
 (segment (start 170.688 77.273998) (end 170.688 76.962) (width 0.25) (layer B.Cu) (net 38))
 (segment (start 170.688 78.486) (end 170.688 77.273998) (width 0.25) (layer B.Cu) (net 38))
 (segment (start 170.561 78.613) (end 170.688 78.486) (width 0.25) (layer B.Cu) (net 38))
 (segment (start 187.198 78.232) (end 186.182 79.248) (width 0.25) (layer B.Cu) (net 38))
 (segment (start 185.42 79.248) (end 186.182 79.248) (width 0.25) (layer B.Cu) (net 38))
 (segment (start 169.512 78.613) (end 168.283002 78.613) (width 0.25) (layer B.Cu) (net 38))
 (segment (start 172.085 77.343) (end 174.912 77.343) (width 0.25) (layer B.Cu) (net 38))
 (segment (start 171.704 77.724) (end 172.085 77.343) (width 0.25) (layer B.Cu) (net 38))
 (segment (start 171.704 79.502) (end 171.704 77.724) (width 0.25) (layer B.Cu) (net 38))
 (segment (start 170.688 80.518) (end 171.704 79.502) (width 0.25) (layer B.Cu) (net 38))
 (segment (start 168.402 80.518) (end 170.688 80.518) (width 0.25) (layer B.Cu) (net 38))
 (segment (start 168.156002 80.272002) (end 168.402 80.518) (width 0.25) (layer B.Cu) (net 38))
 (segment (start 168.156002 78.74) (end 168.156002 80.272002) (width 0.25) (layer B.Cu) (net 38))
 (segment (start 168.283002 78.613) (end 168.156002 78.74) (width 0.25) (layer B.Cu) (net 38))
 (segment (start 167.132 91.274) (end 167.132 92.202) (width 0.25) (layer B.Cu) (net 16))
 (segment (start 167.132 92.202) (end 167.894 92.964) (width 0.25) (layer B.Cu) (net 16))
 (segment (start 167.132 69.43) (end 167.132 70.358) (width 0.25) (layer B.Cu) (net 16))
 (segment (start 167.132 70.358) (end 167.894 71.12) (width 0.25) (layer B.Cu) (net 16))
 (segment (start 169.926 57.785) (end 169.756 57.785) (width 0.25) (layer F.Cu) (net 18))
 (segment (start 169.926 57.785) (end 169.926 58.2041) (width 0.25) (layer F.Cu) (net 18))
 (segment (start 169.672 55.372) (end 169.672 55.288) (width 0.25) (layer B.Cu) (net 19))
 (segment (start 169.926 55.245) (end 169.6798 55.245) (width 0.25) (layer B.Cu) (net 19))
 (segment (start 177.292 57.912) (end 177.376 57.912) (width 0.25) (layer F.Cu) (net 23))
 (segment (start 177.546 57.785) (end 177.546 57.8788) (width 0.25) (layer F.Cu) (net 23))
 (segment (start 177.546 55.245) (end 177.7316 55.245) (width 0.25) (layer B.Cu) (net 24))
 (segment (start 181.356 82.38) (end 184.828 82.38) (width 0.25) (layer B.Cu) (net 33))
 (segment (start 184.828 82.38) (end 185.42 81.788) (width 0.25) (layer B.Cu) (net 33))
 (segment (start 181.356 75.1) (end 183.812 75.1) (width 0.25) (layer B.Cu) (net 34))
 (segment (start 183.812 75.1) (end 185.42 76.708) (width 0.25) (layer B.Cu) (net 34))
 (segment (start 181.356 93.556) (end 184.828 93.556) (width 0.25) (layer B.Cu) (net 30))
 (segment (start 184.828 93.048) (end 185.42 92.456) (width 0.25) (layer B.Cu) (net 30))
 (segment (start 181.356 86.276) (end 183.812 86.276) (width 0.25) (layer B.Cu) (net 31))
 (segment (start 183.812 85.768) (end 185.42 87.376) (width 0.25) (layer B.Cu) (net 31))
 (segment (start 173.04 84.328) (end 169.418 84.328) (width 0.25) (layer B.Cu) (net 3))
 (segment (start 167.706 82.616) (end 167.706 74.168) (width 0.25) (layer B.Cu) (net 3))
 (segment (start 169.418 84.328) (end 167.706 82.616) (width 0.25) (layer B.Cu) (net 3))
 (segment (start 177.546 85.598) (end 177.546 85.09) (width 0.25) (layer B.Cu) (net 4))
 (segment (start 176.784 84.328) (end 177.546 85.09) (width 0.25) (layer B.Cu) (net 4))
 (segment (start 174.94 84.328) (end 176.784 84.328) (width 0.25) (layer B.Cu) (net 4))
 (segment (start 179.832 104.14) (end 185.42 104.14) (width 0.25) (layer B.Cu) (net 4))
 (segment (start 177.546 101.854) (end 179.832 104.14) (width 0.25) (layer B.Cu) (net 4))
 (segment (start 177.546 85.598) (end 177.546 101.854) (width 0.25) (layer B.Cu) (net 4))
 (segment (start 174.94 84.328) (end 174.94 81.181) (width 0.25) (layer B.Cu) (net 4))
 (segment (start 174.94 81.181) (end 174.912 81.153) (width 0.25) (layer B.Cu) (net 4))
 (segment (start 174.912 84.234) (end 174.818 84.328) (width 0.25) (layer B.Cu) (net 4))
 (segment (start 175.039 81.28) (end 174.912 81.153) (width 0.25) (layer B.Cu) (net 4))
 (segment (start 169.606 74.168) (end 169.606 77.249) (width 0.25) (layer B.Cu) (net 5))
 (segment (start 169.606 77.249) (end 169.512 77.343) (width 0.25) (layer B.Cu) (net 5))
 (segment (start 167.132 67.73) (end 167.132 66.802) (width 0.25) (layer B.Cu) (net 28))
 (segment (start 167.132 66.802) (end 167.894 66.04) (width 0.25) (layer B.Cu) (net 28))
 (segment (start 167.132 89.574) (end 167.132 88.646) (width 0.25) (layer B.Cu) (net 17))
 (segment (start 167.132 88.646) (end 167.894 87.884) (width 0.25) (layer B.Cu) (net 17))
 (segment (start 181.356 78.74) (end 179.832 78.74) (width 0.25) (layer B.Cu) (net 32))
 (segment (start 170.561 79.883) (end 169.512 79.883) (width 0.25) (layer B.Cu) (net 32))
 (segment (start 171.196 79.248) (end 170.561 79.883) (width 0.25) (layer B.Cu) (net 32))
 (segment (start 171.196 77.216) (end 171.196 79.248) (width 0.25) (layer B.Cu) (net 32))
 (segment (start 173.228 75.184) (end 171.196 77.216) (width 0.25) (layer B.Cu) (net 32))
 (segment (start 176.276 75.184) (end 173.228 75.184) (width 0.25) (layer B.Cu) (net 32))
 (segment (start 179.832 78.74) (end 176.276 75.184) (width 0.25) (layer B.Cu) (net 32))
 (segment (start 181.356 80.18) (end 181.356 78.74) (width 0.25) (layer B.Cu) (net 32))
 (segment (start 181.356 78.74) (end 181.356 77.3) (width 0.25) (layer B.Cu) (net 32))
 (segment (start 181.356 89.916) (end 179.324 89.916) (width 0.25) (layer B.Cu) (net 29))
 (segment (start 177.165 78.613) (end 174.912 78.613) (width 0.25) (layer B.Cu) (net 29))
 (segment (start 178.308 79.756) (end 177.165 78.613) (width 0.25) (layer B.Cu) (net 29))
 (segment (start 178.308 88.9) (end 178.308 80.264) (width 0.25) (layer B.Cu) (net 29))
 (segment (start 179.324 89.916) (end 178.308 88.9) (width 0.25) (layer B.Cu) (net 29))
 (segment (start 181.356 91.356) (end 181.356 89.916) (width 0.25) (layer B.Cu) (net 29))
 (segment (start 181.356 89.916) (end 181.356 88.476) (width 0.25) (layer B.Cu) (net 29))
 (segment (start 169.512 81.153) (end 169.512 82.71) (width 0.25) (layer B.Cu) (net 36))
 (via (at 169.418 82.804) (size 0.6) (drill 0.4) (layers F.Cu B.Cu) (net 36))
 (segment (start 169.512 82.71) (end 169.418 82.804) (width 0.25) (layer B.Cu) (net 36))
 (segment (start 174.912 79.883) (end 176.657 79.883) (width 0.25) (layer B.Cu) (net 35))
 (via (at 176.784 79.756) (size 0.6) (drill 0.4) (layers F.Cu B.Cu) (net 35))
 (segment (start 176.657 79.883) (end 176.784 79.756) (width 0.25) (layer B.Cu) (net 35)))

